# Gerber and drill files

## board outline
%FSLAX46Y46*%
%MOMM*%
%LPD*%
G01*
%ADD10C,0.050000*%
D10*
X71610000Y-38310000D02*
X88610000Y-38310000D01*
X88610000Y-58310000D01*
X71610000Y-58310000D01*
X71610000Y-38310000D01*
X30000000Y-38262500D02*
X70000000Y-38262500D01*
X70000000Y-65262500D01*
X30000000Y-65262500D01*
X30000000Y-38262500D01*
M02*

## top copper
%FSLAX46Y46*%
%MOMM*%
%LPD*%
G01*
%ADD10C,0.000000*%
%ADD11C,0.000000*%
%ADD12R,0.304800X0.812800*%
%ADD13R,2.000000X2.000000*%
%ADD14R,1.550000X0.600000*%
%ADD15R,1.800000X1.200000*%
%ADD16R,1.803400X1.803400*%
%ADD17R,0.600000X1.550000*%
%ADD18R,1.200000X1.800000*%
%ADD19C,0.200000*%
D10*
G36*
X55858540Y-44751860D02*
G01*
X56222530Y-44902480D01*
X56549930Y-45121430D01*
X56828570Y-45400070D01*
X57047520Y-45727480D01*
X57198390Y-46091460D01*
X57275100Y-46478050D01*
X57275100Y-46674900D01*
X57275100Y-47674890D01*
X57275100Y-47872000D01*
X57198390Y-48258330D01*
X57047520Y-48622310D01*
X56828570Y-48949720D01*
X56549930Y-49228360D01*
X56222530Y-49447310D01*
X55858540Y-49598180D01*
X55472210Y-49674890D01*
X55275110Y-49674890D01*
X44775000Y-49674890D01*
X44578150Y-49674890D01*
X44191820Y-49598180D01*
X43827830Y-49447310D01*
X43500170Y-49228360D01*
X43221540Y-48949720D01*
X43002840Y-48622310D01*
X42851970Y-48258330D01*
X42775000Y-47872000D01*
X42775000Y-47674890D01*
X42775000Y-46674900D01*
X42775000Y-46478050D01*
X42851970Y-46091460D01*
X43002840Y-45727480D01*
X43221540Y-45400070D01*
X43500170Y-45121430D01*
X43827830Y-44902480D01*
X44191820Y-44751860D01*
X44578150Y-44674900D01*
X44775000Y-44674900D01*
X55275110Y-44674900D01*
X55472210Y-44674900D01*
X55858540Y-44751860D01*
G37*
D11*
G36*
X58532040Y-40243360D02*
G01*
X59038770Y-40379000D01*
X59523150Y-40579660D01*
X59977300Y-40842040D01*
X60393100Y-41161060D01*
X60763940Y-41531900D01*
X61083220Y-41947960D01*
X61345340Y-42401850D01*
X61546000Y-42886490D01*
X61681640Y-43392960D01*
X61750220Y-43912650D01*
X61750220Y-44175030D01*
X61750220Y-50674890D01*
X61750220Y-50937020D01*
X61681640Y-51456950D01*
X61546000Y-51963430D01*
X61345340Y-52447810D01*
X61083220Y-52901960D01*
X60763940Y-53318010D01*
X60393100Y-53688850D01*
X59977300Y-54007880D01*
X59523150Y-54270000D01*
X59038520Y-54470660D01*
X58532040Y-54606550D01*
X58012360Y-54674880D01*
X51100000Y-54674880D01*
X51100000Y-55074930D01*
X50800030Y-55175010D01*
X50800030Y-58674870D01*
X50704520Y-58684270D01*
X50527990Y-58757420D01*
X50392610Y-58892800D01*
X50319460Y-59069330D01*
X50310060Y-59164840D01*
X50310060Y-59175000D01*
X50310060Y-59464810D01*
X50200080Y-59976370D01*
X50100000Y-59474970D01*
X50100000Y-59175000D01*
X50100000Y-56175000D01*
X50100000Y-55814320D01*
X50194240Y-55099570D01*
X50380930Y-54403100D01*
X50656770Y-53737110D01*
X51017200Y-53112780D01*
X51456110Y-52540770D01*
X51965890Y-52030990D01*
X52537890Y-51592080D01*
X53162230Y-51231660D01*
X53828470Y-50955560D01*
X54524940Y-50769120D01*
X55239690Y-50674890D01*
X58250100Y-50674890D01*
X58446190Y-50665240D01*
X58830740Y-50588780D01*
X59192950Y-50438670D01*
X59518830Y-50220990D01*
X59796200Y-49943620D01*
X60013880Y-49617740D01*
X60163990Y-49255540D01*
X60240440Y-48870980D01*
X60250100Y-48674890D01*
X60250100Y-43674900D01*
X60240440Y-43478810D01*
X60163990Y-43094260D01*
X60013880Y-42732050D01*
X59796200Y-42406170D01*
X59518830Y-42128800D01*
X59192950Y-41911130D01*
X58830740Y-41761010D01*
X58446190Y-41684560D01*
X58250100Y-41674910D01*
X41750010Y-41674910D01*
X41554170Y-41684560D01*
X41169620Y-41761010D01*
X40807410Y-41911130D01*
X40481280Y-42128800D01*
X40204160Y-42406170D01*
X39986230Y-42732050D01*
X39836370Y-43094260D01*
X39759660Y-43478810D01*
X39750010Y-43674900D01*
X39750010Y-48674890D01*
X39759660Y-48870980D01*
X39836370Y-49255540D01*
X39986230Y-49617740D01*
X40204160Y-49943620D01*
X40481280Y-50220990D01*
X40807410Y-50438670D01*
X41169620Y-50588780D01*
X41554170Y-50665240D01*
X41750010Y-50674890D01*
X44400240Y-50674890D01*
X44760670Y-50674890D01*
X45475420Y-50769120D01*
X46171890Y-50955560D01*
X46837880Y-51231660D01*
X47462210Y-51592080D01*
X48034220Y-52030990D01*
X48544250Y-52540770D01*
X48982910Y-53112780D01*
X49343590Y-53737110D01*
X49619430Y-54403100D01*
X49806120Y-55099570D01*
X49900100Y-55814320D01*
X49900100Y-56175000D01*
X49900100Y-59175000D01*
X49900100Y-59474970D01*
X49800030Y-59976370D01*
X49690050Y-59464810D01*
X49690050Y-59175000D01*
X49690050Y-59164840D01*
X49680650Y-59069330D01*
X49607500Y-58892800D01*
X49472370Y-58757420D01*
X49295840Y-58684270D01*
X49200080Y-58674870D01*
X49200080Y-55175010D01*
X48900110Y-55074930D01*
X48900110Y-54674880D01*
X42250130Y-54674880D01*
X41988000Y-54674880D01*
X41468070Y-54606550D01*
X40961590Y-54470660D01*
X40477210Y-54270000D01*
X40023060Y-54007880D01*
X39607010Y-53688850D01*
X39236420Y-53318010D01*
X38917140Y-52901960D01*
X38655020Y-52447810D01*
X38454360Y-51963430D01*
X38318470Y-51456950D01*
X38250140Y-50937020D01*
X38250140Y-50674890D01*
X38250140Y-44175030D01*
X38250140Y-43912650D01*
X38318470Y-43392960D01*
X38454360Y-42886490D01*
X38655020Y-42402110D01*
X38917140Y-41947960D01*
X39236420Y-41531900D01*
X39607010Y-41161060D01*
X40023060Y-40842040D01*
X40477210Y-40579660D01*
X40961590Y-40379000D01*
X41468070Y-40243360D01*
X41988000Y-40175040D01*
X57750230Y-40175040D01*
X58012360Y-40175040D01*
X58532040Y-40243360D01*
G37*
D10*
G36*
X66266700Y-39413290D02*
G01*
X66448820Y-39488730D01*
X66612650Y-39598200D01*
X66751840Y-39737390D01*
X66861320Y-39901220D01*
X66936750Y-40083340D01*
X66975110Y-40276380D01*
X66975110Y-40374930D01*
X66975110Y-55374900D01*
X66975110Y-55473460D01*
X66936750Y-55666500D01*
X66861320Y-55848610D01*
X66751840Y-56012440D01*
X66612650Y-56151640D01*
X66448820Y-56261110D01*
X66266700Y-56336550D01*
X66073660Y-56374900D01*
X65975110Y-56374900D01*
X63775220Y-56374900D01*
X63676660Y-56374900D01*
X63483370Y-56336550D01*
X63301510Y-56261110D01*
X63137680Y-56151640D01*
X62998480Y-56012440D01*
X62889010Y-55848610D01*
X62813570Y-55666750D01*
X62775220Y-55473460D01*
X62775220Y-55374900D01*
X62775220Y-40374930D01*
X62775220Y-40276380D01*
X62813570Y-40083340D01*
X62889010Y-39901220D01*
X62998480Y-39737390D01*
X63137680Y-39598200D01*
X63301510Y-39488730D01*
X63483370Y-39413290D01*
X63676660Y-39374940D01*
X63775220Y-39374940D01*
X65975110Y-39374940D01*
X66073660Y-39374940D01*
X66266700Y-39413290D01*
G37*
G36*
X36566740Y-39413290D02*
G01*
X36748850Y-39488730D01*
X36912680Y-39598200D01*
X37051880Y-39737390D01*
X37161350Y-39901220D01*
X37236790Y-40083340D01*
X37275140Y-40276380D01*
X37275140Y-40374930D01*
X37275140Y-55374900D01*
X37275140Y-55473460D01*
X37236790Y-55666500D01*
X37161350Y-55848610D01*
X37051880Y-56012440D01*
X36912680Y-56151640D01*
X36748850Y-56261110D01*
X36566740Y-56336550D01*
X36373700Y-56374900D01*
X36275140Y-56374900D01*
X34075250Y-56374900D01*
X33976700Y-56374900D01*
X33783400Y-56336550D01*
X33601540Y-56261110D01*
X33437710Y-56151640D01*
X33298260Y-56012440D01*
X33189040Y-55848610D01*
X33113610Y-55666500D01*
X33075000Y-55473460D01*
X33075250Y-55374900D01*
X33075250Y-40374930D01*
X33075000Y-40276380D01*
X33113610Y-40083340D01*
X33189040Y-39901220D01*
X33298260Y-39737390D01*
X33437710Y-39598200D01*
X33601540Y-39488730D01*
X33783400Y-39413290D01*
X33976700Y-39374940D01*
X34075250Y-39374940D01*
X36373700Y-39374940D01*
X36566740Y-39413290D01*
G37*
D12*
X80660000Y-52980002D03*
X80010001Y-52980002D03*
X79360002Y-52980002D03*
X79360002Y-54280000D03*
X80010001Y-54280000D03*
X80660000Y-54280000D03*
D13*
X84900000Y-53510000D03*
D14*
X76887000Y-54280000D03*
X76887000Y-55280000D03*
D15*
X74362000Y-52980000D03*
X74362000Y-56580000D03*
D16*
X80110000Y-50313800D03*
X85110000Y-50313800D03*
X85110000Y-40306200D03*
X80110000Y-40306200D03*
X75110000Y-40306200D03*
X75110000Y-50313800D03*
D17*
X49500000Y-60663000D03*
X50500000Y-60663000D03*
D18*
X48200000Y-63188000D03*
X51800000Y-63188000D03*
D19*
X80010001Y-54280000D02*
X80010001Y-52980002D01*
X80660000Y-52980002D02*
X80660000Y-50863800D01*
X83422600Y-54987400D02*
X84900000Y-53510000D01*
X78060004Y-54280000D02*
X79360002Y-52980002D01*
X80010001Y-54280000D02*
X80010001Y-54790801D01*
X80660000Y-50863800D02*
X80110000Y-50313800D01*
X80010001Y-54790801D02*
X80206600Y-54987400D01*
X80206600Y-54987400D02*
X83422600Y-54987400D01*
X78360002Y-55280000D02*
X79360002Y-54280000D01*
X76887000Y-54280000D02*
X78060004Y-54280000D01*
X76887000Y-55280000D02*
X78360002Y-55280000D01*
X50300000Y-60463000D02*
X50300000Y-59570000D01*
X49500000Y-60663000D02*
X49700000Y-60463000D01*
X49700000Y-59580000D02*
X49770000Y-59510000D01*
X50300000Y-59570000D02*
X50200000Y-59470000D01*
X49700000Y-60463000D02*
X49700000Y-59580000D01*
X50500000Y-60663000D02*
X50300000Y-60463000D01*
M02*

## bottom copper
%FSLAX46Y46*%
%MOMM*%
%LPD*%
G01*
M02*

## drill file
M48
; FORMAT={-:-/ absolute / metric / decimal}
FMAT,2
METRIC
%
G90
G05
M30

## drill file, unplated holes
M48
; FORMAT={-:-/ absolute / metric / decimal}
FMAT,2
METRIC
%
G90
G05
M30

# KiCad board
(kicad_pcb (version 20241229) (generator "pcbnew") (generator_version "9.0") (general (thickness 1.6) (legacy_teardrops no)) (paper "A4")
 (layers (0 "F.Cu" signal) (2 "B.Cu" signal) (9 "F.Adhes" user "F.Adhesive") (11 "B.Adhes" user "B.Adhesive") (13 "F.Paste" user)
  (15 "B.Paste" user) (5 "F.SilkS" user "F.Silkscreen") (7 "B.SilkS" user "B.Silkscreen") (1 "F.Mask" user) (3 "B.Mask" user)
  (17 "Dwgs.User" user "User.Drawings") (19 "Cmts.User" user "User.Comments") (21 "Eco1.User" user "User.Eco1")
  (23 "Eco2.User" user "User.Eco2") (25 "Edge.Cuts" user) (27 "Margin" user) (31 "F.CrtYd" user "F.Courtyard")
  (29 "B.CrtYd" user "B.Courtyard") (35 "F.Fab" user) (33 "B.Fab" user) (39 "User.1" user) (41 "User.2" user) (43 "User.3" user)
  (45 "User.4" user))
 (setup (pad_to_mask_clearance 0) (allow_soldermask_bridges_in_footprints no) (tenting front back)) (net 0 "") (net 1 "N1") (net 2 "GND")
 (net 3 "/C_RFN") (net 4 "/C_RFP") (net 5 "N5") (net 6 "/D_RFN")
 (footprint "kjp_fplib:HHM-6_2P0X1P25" (layer "F.Cu") (at 80.010001 53.630001 -90)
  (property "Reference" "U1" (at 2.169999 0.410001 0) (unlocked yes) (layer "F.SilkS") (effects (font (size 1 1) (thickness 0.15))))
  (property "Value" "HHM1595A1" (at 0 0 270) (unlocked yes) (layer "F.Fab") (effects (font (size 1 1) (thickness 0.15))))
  (pad "1" smd rect (at -0.649999 -0.649999 270) (size 0.8128 0.3048) (layers "F.Cu" "F.Mask" "F.Paste") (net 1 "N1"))
  (pad "2" smd rect (at -0.649999 0 270) (size 0.8128 0.3048) (layers "F.Cu" "F.Mask" "F.Paste") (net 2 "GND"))
  (pad "3" smd rect (at -0.649999 0.649999 270) (size 0.8128 0.3048) (layers "F.Cu" "F.Mask" "F.Paste") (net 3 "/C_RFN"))
  (pad "4" smd rect (at 0.649999 0.649999 270) (size 0.8128 0.3048) (layers "F.Cu" "F.Mask" "F.Paste") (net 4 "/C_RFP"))
  (pad "5" smd rect (at 0.649999 0 270) (size 0.8128 0.3048) (layers "F.Cu" "F.Mask" "F.Paste") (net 2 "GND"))
  (pad "6" smd rect (at 0.649999 -0.649999 270) (size 0.8128 0.3048) (layers "F.Cu" "F.Mask" "F.Paste") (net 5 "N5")))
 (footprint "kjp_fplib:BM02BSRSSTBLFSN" (layer "F.Cu") (at 75.05 54.78 -90)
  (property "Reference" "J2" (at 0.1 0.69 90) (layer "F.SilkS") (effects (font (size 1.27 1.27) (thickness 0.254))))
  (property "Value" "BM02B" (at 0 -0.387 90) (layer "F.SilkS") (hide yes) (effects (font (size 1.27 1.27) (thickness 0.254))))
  (pad "1" smd rect (at -0.5 -1.837 270) (size 0.6 1.55) (layers "F.Cu" "F.Mask" "F.Paste") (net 3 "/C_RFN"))
  (pad "2" smd rect (at 0.5 -1.837 270) (size 0.6 1.55) (layers "F.Cu" "F.Mask" "F.Paste") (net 4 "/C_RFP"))
  (pad "MP1" smd rect (at -1.8 0.688 270) (size 1.2 1.8) (layers "F.Cu" "F.Mask" "F.Paste"))
  (pad "MP2" smd rect (at 1.8 0.688 270) (size 1.2 1.8) (layers "F.Cu" "F.Mask" "F.Paste")))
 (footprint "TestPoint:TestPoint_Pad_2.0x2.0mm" (layer "F.Cu") (at 84.9 53.51)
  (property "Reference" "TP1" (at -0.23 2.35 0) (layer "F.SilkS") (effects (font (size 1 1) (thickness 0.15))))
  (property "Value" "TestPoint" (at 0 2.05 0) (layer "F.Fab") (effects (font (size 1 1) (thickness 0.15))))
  (pad "1" smd rect (at 0 0) (size 2 2) (layers "F.Cu" "F.Mask") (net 2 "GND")))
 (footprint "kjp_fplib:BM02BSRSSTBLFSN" (layer "F.Cu") (at 50 62.5)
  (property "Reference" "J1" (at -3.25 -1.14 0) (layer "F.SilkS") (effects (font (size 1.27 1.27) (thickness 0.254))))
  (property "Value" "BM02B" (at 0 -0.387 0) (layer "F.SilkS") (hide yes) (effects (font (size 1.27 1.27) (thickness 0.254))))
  (pad "1" smd rect (at -0.5 -1.837) (size 0.6 1.55) (layers "F.Cu" "F.Mask" "F.Paste") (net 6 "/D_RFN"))
  (pad "2" smd rect (at 0.5 -1.837) (size 0.6 1.55) (layers "F.Cu" "F.Mask" "F.Paste") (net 6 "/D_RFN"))
  (pad "MP1" smd rect (at -1.8 0.688) (size 1.2 1.8) (layers "F.Cu" "F.Mask" "F.Paste"))
  (pad "MP2" smd rect (at 1.8 0.688) (size 1.2 1.8) (layers "F.Cu" "F.Mask" "F.Paste")))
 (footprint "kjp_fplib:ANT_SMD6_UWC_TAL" (layer "F.Cu") (at 80.11 45.31 90)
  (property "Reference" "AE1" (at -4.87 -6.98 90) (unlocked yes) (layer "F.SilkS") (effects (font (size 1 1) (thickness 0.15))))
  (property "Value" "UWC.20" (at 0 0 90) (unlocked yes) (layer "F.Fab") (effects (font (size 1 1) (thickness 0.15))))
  (pad "1" smd rect (at -5.0038 0 90) (size 1.8034 1.8034) (layers "F.Cu" "F.Mask" "F.Paste") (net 1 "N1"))
  (pad "2" smd rect (at -5.0038 5 90) (size 1.8034 1.8034) (layers "F.Cu" "F.Mask" "F.Paste"))
  (pad "3" smd rect (at 5.0038 5 90) (size 1.8034 1.8034) (layers "F.Cu" "F.Mask" "F.Paste"))
  (pad "4" smd rect (at 5.0038 0 90) (size 1.8034 1.8034) (layers "F.Cu" "F.Mask" "F.Paste"))
  (pad "5" smd rect (at 5.0038 -5 90) (size 1.8034 1.8034) (layers "F.Cu" "F.Mask" "F.Paste"))
  (pad "6" smd rect (at -5.0038 -5 90) (size 1.8034 1.8034) (layers "F.Cu" "F.Mask" "F.Paste")))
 (gr_poly
  (pts (xy 36.56674 39.41329) (xy 36.74885 39.48873) (xy 36.91268 39.5982) (xy 37.05188 39.73739) (xy 37.16135 39.90122)
   (xy 37.23679 40.08334) (xy 37.27514 40.27638) (xy 37.27514 40.37493) (xy 37.27514 55.3749) (xy 37.27514 55.47346) (xy 37.23679 55.6665)
   (xy 37.16135 55.84861) (xy 37.05188 56.01244) (xy 36.91268 56.15164) (xy 36.74885 56.26111) (xy 36.56674 56.33655) (xy 36.3737 56.3749)
   (xy 36.27514 56.3749) (xy 34.07525 56.3749) (xy 33.9767 56.3749) (xy 33.7834 56.33655) (xy 33.60154 56.26111) (xy 33.43771 56.15164)
   (xy 33.29826 56.01244) (xy 33.18904 55.84861) (xy 33.11361 55.6665) (xy 33.075 55.47346) (xy 33.07525 55.3749) (xy 33.07525 40.37493)
   (xy 33.075 40.27638) (xy 33.11361 40.08334) (xy 33.18904 39.90122) (xy 33.29826 39.73739) (xy 33.43771 39.5982) (xy 33.60154 39.48873)
   (xy 33.7834 39.41329) (xy 33.9767 39.37494) (xy 34.07525 39.37494) (xy 36.3737 39.37494))
  (stroke (width 0) (type solid)) (fill yes) (layer "F.Cu"))
 (gr_poly
  (pts (xy 65.97511 39.37494) (xy 66.07366 39.37494) (xy 66.2667 39.41329) (xy 66.44882 39.48873) (xy 66.61265 39.5982)
   (xy 66.75184 39.73739) (xy 66.86132 39.90122) (xy 66.93675 40.08334) (xy 66.97511 40.27638) (xy 66.97511 40.37493) (xy 66.97511 55.3749)
   (xy 66.97511 55.47346) (xy 66.93675 55.6665) (xy 66.86132 55.84861) (xy 66.75184 56.01244) (xy 66.61265 56.15164) (xy 66.44882 56.26111)
   (xy 66.2667 56.33655) (xy 66.07366 56.3749) (xy 65.97511 56.3749) (xy 63.77522 56.3749) (xy 63.67666 56.3749) (xy 63.48337 56.33655)
   (xy 63.30151 56.26111) (xy 63.13768 56.15164) (xy 62.99848 56.01244) (xy 62.88901 55.84861) (xy 62.81357 55.66675) (xy 62.77522 55.47346)
   (xy 62.77522 55.3749) (xy 62.77522 40.37493) (xy 62.77522 40.27638) (xy 62.81357 40.08334) (xy 62.88901 39.90122) (xy 62.99848 39.73739)
   (xy 63.13768 39.5982) (xy 63.30151 39.48873) (xy 63.48337 39.41329) (xy 63.67666 39.37494) (xy 63.77522 39.37494))
  (stroke (width 0) (type solid)) (fill yes) (layer "F.Cu"))
 (gr_poly
  (pts (xy 58.53204 40.24336) (xy 59.03877 40.379) (xy 59.52315 40.57966) (xy 59.9773 40.84204) (xy 60.3931 41.16106) (xy 60.76394 41.5319)
   (xy 61.08322 41.94796) (xy 61.34534 42.40185) (xy 61.546 42.88649) (xy 61.68164 43.39296) (xy 61.75022 43.91265) (xy 61.75022 44.17503)
   (xy 61.75022 50.67489) (xy 61.75022 50.93702) (xy 61.68164 51.45695) (xy 61.546 51.96343) (xy 61.34534 52.44781) (xy 61.08322 52.90196)
   (xy 60.76394 53.31801) (xy 60.3931 53.68885) (xy 59.9773 54.00788) (xy 59.52315 54.27) (xy 59.03852 54.47066) (xy 58.53204 54.60655)
   (xy 58.01236 54.67488) (xy 51.1 54.67488) (xy 51.1 55.07493) (xy 50.80003 55.17501) (xy 50.80003 58.67487) (xy 50.70452 58.68427)
   (xy 50.52799 58.75742) (xy 50.39261 58.8928) (xy 50.31946 59.06933) (xy 50.31006 59.16484) (xy 50.31006 59.175) (xy 50.31006 59.46481)
   (xy 50.20008 59.97637) (xy 50.1 59.47497) (xy 50.1 59.175) (xy 50.1 56.175) (xy 50.1 55.81432) (xy 50.19424 55.09957)
   (xy 50.38093 54.4031) (xy 50.65677 53.73711) (xy 51.0172 53.11278) (xy 51.45611 52.54077) (xy 51.96589 52.03099) (xy 52.53789 51.59208)
   (xy 53.16223 51.23166) (xy 53.82847 50.95556) (xy 54.52494 50.76912) (xy 55.23969 50.67489) (xy 58.2501 50.67489) (xy 58.44619 50.66524)
   (xy 58.83074 50.58878) (xy 59.19295 50.43867) (xy 59.51883 50.22099) (xy 59.7962 49.94362) (xy 60.01388 49.61774) (xy 60.16399 49.25554)
   (xy 60.24044 48.87098) (xy 60.2501 48.67489) (xy 60.2501 43.6749) (xy 60.24044 43.47881) (xy 60.16399 43.09426) (xy 60.01388 42.73205)
   (xy 59.7962 42.40617) (xy 59.51883 42.1288) (xy 59.19295 41.91113) (xy 58.83074 41.76101) (xy 58.44619 41.68456) (xy 58.2501 41.67491)
   (xy 41.75001 41.67491) (xy 41.55417 41.68456) (xy 41.16962 41.76101) (xy 40.80741 41.91113) (xy 40.48128 42.1288) (xy 40.20416 42.40617)
   (xy 39.98623 42.73205) (xy 39.83637 43.09426) (xy 39.75966 43.47881) (xy 39.75001 43.6749) (xy 39.75001 48.67489) (xy 39.75966 48.87098)
   (xy 39.83637 49.25554) (xy 39.98623 49.61774) (xy 40.20416 49.94362) (xy 40.48128 50.22099) (xy 40.80741 50.43867) (xy 41.16962 50.58878)
   (xy 41.55417 50.66524) (xy 41.75001 50.67489) (xy 44.40024 50.67489) (xy 44.76067 50.67489) (xy 45.47542 50.76912) (xy 46.17189 50.95556)
   (xy 46.83788 51.23166) (xy 47.46221 51.59208) (xy 48.03422 52.03099) (xy 48.54425 52.54077) (xy 48.98291 53.11278) (xy 49.34359 53.73711)
   (xy 49.61943 54.4031) (xy 49.80612 55.09957) (xy 49.9001 55.81432) (xy 49.9001 56.175) (xy 49.9001 59.175) (xy 49.9001 59.47497)
   (xy 49.80003 59.97637) (xy 49.69005 59.46481) (xy 49.69005 59.175) (xy 49.69005 59.16484) (xy 49.68065 59.06933) (xy 49.6075 58.8928)
   (xy 49.47237 58.75742) (xy 49.29584 58.68427) (xy 49.20008 58.67487) (xy 49.20008 55.17501) (xy 48.90011 55.07493) (xy 48.90011 54.67488)
   (xy 42.25013 54.67488) (xy 41.988 54.67488) (xy 41.46807 54.60655) (xy 40.96159 54.47066) (xy 40.47721 54.27) (xy 40.02306 54.00788)
   (xy 39.60701 53.68885) (xy 39.23642 53.31801) (xy 38.91714 52.90196) (xy 38.65502 52.44781) (xy 38.45436 51.96343) (xy 38.31847 51.45695)
   (xy 38.25014 50.93702) (xy 38.25014 50.67489) (xy 38.25014 44.17503) (xy 38.25014 43.91265) (xy 38.31847 43.39296) (xy 38.45436 42.88649)
   (xy 38.65502 42.40211) (xy 38.91714 41.94796) (xy 39.23642 41.5319) (xy 39.60701 41.16106) (xy 40.02306 40.84204) (xy 40.47721 40.57966)
   (xy 40.96159 40.379) (xy 41.46807 40.24336) (xy 41.988 40.17504) (xy 57.75023 40.17504) (xy 58.01236 40.17504))
  (stroke (width 0) (type solid)) (fill yes) (layer "F.Cu") (net 6))
 (gr_poly
  (pts (xy 55.85854 44.75186) (xy 56.22253 44.90248) (xy 56.54993 45.12143) (xy 56.82857 45.40007) (xy 57.04752 45.72748)
   (xy 57.19839 46.09146) (xy 57.2751 46.47805) (xy 57.2751 46.6749) (xy 57.2751 47.67489) (xy 57.2751 47.872) (xy 57.19839 48.25833)
   (xy 57.04752 48.62231) (xy 56.82857 48.94972) (xy 56.54993 49.22836) (xy 56.22253 49.44731) (xy 55.85854 49.59818) (xy 55.47221 49.67489)
   (xy 55.27511 49.67489) (xy 44.775 49.67489) (xy 44.57815 49.67489) (xy 44.19182 49.59818) (xy 43.82783 49.44731) (xy 43.50017 49.22836)
   (xy 43.22154 48.94972) (xy 43.00284 48.62231) (xy 42.85197 48.25833) (xy 42.775 47.872) (xy 42.775 47.67489) (xy 42.775 46.6749)
   (xy 42.775 46.47805) (xy 42.85197 46.09146) (xy 43.00284 45.72748) (xy 43.22154 45.40007) (xy 43.50017 45.12143) (xy 43.82783 44.90248)
   (xy 44.19182 44.75186) (xy 44.57815 44.6749) (xy 44.775 44.6749) (xy 55.27511 44.6749) (xy 55.47221 44.6749))
  (stroke (width 0) (type solid)) (fill yes) (layer "F.Cu"))
 (gr_rect (start 30 38.2625) (end 70 65.2625) (stroke (width 0.05) (type solid)) (fill no) (layer "Edge.Cuts"))
 (gr_rect (start 71.61 38.31) (end 88.61 58.31) (stroke (width 0.05) (type solid)) (fill no) (layer "Edge.Cuts"))
 (segment (start 80.66 50.8638) (end 80.11 50.3138) (width 0.2) (layer "F.Cu") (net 1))
 (segment (start 80.66 52.980002) (end 80.66 50.8638) (width 0.2) (layer "F.Cu") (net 1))
 (segment (start 49.5 60.663) (end 49.7 60.463) (width 0.2) (layer "F.Cu") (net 6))
 (segment (start 49.7 60.463) (end 49.7 59.58) (width 0.2) (layer "F.Cu") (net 6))
 (segment (start 50.3 60.463) (end 50.3 59.57) (width 0.2) (layer "F.Cu") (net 6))
 (segment (start 50.3 59.57) (end 50.2 59.47) (width 0.2) (layer "F.Cu") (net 6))
 (segment (start 50.5 60.663) (end 50.3 60.463) (width 0.2) (layer "F.Cu") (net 6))
 (segment (start 49.7 59.58) (end 49.77 59.51) (width 0.2) (layer "F.Cu") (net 6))
 (segment (start 78.360002 55.28) (end 79.360002 54.28) (width 0.2) (layer "F.Cu") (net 4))
 (segment (start 76.887 55.28) (end 78.360002 55.28) (width 0.2) (layer "F.Cu") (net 4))
 (segment (start 76.887 54.28) (end 78.060004 54.28) (width 0.2) (layer "F.Cu") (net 3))
 (segment (start 78.060004 54.28) (end 79.360002 52.980002) (width 0.2) (layer "F.Cu") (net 3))
 (segment (start 80.010001 54.790801) (end 80.2066 54.9874) (width 0.2) (layer "F.Cu") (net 2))
 (segment (start 80.2066 54.9874) (end 83.4226 54.9874) (width 0.2) (layer "F.Cu") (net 2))
 (segment (start 80.010001 54.28) (end 80.010001 54.790801) (width 0.2) (layer "F.Cu") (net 2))
 (segment (start 80.010001 54.28) (end 80.010001 52.980002) (width 0.2) (layer "F.Cu") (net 2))
 (segment (start 83.4226 54.9874) (end 84.9 53.51) (width 0.2) (layer "F.Cu") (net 2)))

